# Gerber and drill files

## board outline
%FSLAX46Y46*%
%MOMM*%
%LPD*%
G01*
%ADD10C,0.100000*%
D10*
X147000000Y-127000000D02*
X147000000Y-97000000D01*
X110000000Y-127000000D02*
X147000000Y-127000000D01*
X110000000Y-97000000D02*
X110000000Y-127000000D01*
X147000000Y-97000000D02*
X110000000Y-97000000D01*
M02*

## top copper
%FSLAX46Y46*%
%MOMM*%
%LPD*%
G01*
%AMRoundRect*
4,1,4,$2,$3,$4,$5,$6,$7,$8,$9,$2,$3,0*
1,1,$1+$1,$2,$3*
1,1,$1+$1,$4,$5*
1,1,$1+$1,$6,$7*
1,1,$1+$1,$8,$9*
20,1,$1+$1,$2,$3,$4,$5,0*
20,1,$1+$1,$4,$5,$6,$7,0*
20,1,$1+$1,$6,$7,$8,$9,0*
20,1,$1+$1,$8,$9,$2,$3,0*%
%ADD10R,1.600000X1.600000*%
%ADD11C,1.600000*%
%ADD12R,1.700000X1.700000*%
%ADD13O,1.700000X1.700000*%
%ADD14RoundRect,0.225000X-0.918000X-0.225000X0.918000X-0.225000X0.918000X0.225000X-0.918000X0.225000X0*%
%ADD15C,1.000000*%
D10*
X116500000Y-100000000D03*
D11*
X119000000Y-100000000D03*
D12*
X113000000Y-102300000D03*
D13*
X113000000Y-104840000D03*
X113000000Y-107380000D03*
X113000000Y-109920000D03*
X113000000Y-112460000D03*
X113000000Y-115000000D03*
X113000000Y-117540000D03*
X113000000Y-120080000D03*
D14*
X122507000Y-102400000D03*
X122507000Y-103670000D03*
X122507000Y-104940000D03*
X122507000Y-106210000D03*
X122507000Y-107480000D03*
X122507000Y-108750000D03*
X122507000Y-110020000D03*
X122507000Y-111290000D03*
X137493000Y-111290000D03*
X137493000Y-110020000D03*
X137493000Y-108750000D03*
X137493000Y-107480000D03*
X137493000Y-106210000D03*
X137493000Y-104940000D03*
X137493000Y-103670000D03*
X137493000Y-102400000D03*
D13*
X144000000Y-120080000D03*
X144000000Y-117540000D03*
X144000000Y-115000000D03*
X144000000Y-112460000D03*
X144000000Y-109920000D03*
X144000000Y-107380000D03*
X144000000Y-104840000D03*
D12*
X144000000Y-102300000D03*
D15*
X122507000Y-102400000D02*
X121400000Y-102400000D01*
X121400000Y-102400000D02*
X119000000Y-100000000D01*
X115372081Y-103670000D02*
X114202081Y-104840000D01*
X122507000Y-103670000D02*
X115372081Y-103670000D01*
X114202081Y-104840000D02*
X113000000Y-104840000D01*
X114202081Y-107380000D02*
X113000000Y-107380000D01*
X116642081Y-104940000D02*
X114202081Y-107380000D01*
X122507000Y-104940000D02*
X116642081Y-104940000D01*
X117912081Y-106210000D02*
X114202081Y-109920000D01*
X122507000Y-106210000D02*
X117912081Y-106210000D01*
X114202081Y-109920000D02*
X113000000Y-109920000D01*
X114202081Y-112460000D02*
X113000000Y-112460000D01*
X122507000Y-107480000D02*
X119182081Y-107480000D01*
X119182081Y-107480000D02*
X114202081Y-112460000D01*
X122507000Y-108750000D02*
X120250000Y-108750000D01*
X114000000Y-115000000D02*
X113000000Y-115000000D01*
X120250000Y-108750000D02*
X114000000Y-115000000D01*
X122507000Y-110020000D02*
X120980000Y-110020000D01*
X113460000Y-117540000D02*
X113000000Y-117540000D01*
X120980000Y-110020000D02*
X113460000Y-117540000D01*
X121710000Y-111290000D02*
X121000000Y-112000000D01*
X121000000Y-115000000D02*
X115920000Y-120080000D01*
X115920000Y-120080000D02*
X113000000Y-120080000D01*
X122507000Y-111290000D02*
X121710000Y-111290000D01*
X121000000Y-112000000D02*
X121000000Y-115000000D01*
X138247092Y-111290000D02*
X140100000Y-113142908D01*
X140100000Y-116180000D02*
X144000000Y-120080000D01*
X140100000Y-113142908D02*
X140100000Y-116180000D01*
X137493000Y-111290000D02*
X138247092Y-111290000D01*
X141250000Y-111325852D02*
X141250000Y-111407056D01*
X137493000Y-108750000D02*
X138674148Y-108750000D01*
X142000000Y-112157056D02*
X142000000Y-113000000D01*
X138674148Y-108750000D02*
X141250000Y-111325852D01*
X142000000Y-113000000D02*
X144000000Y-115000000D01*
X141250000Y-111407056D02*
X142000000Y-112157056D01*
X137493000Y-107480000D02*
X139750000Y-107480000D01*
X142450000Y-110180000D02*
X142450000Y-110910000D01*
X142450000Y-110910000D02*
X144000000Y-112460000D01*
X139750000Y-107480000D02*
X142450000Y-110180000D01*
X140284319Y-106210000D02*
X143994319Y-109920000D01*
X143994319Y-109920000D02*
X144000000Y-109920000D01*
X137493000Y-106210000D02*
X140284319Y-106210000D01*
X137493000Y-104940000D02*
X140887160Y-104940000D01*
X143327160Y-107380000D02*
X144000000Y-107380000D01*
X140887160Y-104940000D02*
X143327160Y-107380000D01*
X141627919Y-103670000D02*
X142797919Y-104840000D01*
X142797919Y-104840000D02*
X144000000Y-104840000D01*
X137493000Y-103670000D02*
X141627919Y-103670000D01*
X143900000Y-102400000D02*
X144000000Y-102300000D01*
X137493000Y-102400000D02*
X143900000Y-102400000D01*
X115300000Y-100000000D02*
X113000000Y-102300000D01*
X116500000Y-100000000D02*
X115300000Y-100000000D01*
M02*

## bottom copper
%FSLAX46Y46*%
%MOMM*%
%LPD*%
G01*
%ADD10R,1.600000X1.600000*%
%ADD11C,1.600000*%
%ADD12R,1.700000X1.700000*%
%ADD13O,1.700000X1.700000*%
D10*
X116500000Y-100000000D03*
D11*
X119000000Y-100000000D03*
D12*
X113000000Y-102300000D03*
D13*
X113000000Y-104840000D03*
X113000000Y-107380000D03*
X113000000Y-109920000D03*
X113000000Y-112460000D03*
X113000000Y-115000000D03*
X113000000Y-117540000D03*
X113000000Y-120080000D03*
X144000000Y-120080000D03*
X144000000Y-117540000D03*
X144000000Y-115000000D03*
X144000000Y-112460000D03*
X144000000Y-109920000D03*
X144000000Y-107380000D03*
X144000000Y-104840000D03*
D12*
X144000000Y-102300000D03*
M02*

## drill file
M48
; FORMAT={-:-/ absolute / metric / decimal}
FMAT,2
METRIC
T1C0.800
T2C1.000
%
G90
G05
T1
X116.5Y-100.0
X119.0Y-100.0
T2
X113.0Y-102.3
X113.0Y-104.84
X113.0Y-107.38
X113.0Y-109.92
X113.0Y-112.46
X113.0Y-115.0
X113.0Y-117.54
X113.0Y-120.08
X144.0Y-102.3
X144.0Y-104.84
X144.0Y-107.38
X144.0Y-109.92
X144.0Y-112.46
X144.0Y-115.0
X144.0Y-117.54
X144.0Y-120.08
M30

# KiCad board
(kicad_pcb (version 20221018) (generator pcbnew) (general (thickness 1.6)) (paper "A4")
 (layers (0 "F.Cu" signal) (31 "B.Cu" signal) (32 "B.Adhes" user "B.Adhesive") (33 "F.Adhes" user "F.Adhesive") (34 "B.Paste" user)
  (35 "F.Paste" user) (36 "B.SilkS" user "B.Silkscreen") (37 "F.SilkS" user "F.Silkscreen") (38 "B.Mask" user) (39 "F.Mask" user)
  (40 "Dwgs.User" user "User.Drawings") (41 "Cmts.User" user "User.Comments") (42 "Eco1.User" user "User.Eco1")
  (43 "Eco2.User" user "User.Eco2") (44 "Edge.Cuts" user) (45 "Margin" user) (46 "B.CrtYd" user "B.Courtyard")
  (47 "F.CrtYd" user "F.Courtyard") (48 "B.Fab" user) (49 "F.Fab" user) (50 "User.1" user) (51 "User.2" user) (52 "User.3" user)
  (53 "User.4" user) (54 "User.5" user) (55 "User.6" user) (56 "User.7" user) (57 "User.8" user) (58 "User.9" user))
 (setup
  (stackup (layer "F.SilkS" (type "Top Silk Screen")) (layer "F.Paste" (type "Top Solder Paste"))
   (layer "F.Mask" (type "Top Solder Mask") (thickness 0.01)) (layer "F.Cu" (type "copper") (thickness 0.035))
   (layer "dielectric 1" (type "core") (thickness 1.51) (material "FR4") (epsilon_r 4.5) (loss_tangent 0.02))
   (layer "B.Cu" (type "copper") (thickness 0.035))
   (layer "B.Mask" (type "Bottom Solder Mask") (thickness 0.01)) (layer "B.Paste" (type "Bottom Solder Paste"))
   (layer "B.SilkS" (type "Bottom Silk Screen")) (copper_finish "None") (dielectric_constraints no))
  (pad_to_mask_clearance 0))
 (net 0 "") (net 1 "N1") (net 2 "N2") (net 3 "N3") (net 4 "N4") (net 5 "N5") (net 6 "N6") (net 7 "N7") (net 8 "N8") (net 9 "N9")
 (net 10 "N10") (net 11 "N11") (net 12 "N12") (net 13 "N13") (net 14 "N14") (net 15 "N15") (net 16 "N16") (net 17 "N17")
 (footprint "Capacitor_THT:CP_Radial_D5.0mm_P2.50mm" (layer "F.Cu") (at 116.5 100)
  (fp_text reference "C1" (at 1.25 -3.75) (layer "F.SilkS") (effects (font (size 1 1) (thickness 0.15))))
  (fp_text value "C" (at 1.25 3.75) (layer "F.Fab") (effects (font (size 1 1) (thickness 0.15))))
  (pad "1" thru_hole rect (at 0 0) (size 1.6 1.6) (drill 0.8) (layers "*.Cu" "*.Mask") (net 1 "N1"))
  (pad "2" thru_hole circle (at 2.5 0) (size 1.6 1.6) (drill 0.8) (layers "*.Cu" "*.Mask") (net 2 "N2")))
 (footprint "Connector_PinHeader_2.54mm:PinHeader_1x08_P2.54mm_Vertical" (layer "F.Cu") (at 113 102.3)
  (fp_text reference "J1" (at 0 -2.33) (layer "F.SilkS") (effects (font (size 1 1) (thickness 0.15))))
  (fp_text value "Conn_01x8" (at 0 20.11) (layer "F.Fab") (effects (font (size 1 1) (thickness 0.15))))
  (pad "1" thru_hole rect (at 0 0) (size 1.7 1.7) (drill 1) (layers "*.Cu" "*.Mask") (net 1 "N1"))
  (pad "2" thru_hole oval (at 0 2.54) (size 1.7 1.7) (drill 1) (layers "*.Cu" "*.Mask") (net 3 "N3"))
  (pad "3" thru_hole oval (at 0 5.08) (size 1.7 1.7) (drill 1) (layers "*.Cu" "*.Mask") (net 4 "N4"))
  (pad "4" thru_hole oval (at 0 7.62) (size 1.7 1.7) (drill 1) (layers "*.Cu" "*.Mask") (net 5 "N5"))
  (pad "5" thru_hole oval (at 0 10.16) (size 1.7 1.7) (drill 1) (layers "*.Cu" "*.Mask") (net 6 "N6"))
  (pad "6" thru_hole oval (at 0 12.7) (size 1.7 1.7) (drill 1) (layers "*.Cu" "*.Mask") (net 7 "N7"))
  (pad "7" thru_hole oval (at 0 15.24) (size 1.7 1.7) (drill 1) (layers "*.Cu" "*.Mask") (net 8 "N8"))
  (pad "8" thru_hole oval (at 0 17.78) (size 1.7 1.7) (drill 1) (layers "*.Cu" "*.Mask") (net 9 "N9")))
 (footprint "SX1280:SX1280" (layer "F.Cu") (at 130.493 95.52)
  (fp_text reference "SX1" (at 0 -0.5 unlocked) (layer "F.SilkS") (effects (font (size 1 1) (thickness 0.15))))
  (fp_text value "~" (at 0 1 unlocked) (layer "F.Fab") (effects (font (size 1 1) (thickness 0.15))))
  (pad "1" smd roundrect (at -7.986 6.88) (size 2.286 0.9) (layers "F.Cu" "F.Paste" "F.Mask") (roundrect_rratio 0.25) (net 2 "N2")
   (thermal_bridge_angle 45))
  (pad "2" smd roundrect (at -7.986 8.15) (size 2.286 0.9) (layers "F.Cu" "F.Paste" "F.Mask") (roundrect_rratio 0.25) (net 3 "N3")
   (thermal_bridge_angle 45))
  (pad "3" smd roundrect (at -7.986 9.42) (size 2.286 0.9) (layers "F.Cu" "F.Paste" "F.Mask") (roundrect_rratio 0.25) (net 4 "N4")
   (thermal_bridge_angle 45))
  (pad "4" smd roundrect (at -7.986 10.69) (size 2.286 0.9) (layers "F.Cu" "F.Paste" "F.Mask") (roundrect_rratio 0.25) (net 5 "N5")
   (thermal_bridge_angle 45))
  (pad "5" smd roundrect (at -7.986 11.96) (size 2.286 0.9) (layers "F.Cu" "F.Paste" "F.Mask") (roundrect_rratio 0.25) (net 6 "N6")
   (thermal_bridge_angle 45))
  (pad "6" smd roundrect (at -7.986 13.23) (size 2.286 0.9) (layers "F.Cu" "F.Paste" "F.Mask") (roundrect_rratio 0.25) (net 7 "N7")
   (thermal_bridge_angle 45))
  (pad "7" smd roundrect (at -7.986 14.5) (size 2.286 0.9) (layers "F.Cu" "F.Paste" "F.Mask") (roundrect_rratio 0.25) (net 8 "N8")
   (thermal_bridge_angle 45))
  (pad "8" smd roundrect (at -7.986 15.77) (size 2.286 0.9) (layers "F.Cu" "F.Paste" "F.Mask") (roundrect_rratio 0.25) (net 9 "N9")
   (thermal_bridge_angle 45))
  (pad "9" smd roundrect (at 7 15.77) (size 2.286 0.9) (layers "F.Cu" "F.Paste" "F.Mask") (roundrect_rratio 0.25) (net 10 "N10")
   (thermal_bridge_angle 45))
  (pad "10" smd roundrect (at 7 14.5) (size 2.286 0.9) (layers "F.Cu" "F.Paste" "F.Mask") (roundrect_rratio 0.25) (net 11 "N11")
   (thermal_bridge_angle 45))
  (pad "11" smd roundrect (at 7 13.23) (size 2.286 0.9) (layers "F.Cu" "F.Paste" "F.Mask") (roundrect_rratio 0.25) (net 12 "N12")
   (thermal_bridge_angle 45))
  (pad "12" smd roundrect (at 7 11.96) (size 2.286 0.9) (layers "F.Cu" "F.Paste" "F.Mask") (roundrect_rratio 0.25) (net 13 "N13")
   (thermal_bridge_angle 45))
  (pad "13" smd roundrect (at 7 10.69) (size 2.286 0.9) (layers "F.Cu" "F.Paste" "F.Mask") (roundrect_rratio 0.25) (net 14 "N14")
   (thermal_bridge_angle 45))
  (pad "14" smd roundrect (at 7 9.42) (size 2.286 0.9) (layers "F.Cu" "F.Paste" "F.Mask") (roundrect_rratio 0.25) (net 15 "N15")
   (thermal_bridge_angle 45))
  (pad "15" smd roundrect (at 7 8.15) (size 2.286 0.9) (layers "F.Cu" "F.Paste" "F.Mask") (roundrect_rratio 0.25) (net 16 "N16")
   (thermal_bridge_angle 45))
  (pad "16" smd roundrect (at 7 6.88) (size 2.286 0.9) (layers "F.Cu" "F.Paste" "F.Mask") (roundrect_rratio 0.25) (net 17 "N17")
   (thermal_bridge_angle 45)))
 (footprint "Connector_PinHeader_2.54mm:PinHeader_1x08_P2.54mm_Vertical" (layer "F.Cu") (at 144 102.3)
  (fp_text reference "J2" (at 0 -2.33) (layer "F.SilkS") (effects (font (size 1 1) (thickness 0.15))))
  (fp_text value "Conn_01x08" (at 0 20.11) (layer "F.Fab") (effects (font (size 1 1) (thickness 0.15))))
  (pad "9" thru_hole oval (at 0 17.78) (size 1.7 1.7) (drill 1) (layers "*.Cu" "*.Mask") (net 10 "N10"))
  (pad "10" thru_hole oval (at 0 15.24) (size 1.7 1.7) (drill 1) (layers "*.Cu" "*.Mask") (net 11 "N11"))
  (pad "11" thru_hole oval (at 0 12.7) (size 1.7 1.7) (drill 1) (layers "*.Cu" "*.Mask") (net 12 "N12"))
  (pad "12" thru_hole oval (at 0 10.16) (size 1.7 1.7) (drill 1) (layers "*.Cu" "*.Mask") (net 13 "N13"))
  (pad "13" thru_hole oval (at 0 7.62) (size 1.7 1.7) (drill 1) (layers "*.Cu" "*.Mask") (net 14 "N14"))
  (pad "14" thru_hole oval (at 0 5.08) (size 1.7 1.7) (drill 1) (layers "*.Cu" "*.Mask") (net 15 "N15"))
  (pad "15" thru_hole oval (at 0 2.54) (size 1.7 1.7) (drill 1) (layers "*.Cu" "*.Mask") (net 16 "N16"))
  (pad "16" thru_hole rect (at 0 0) (size 1.7 1.7) (drill 1) (layers "*.Cu" "*.Mask") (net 17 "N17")))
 (gr_line (start 147 127) (end 147 97) (stroke (width 0.1) (type default)) (layer "Edge.Cuts"))
 (gr_line (start 110 127) (end 147 127) (stroke (width 0.1) (type default)) (layer "Edge.Cuts"))
 (gr_line (start 110 97) (end 110 127) (stroke (width 0.1) (type default)) (layer "Edge.Cuts"))
 (gr_line (start 147 97) (end 110 97) (stroke (width 0.1) (type default)) (layer "Edge.Cuts"))
 (segment (start 122.507 102.4) (end 121.4 102.4) (width 1) (layer "F.Cu") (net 2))
 (segment (start 121.4 102.4) (end 119 100) (width 1) (layer "F.Cu") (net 2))
 (segment (start 115.372081 103.67) (end 114.202081 104.84) (width 1) (layer "F.Cu") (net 3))
 (segment (start 122.507 103.67) (end 115.372081 103.67) (width 1) (layer "F.Cu") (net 3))
 (segment (start 114.202081 104.84) (end 113 104.84) (width 1) (layer "F.Cu") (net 3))
 (segment (start 114.202081 107.38) (end 113 107.38) (width 1) (layer "F.Cu") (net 4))
 (segment (start 116.642081 104.94) (end 114.202081 107.38) (width 1) (layer "F.Cu") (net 4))
 (segment (start 122.507 104.94) (end 116.642081 104.94) (width 1) (layer "F.Cu") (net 4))
 (segment (start 117.912081 106.21) (end 114.202081 109.92) (width 1) (layer "F.Cu") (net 5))
 (segment (start 122.507 106.21) (end 117.912081 106.21) (width 1) (layer "F.Cu") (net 5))
 (segment (start 114.202081 109.92) (end 113 109.92) (width 1) (layer "F.Cu") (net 5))
 (segment (start 114.202081 112.46) (end 113 112.46) (width 1) (layer "F.Cu") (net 6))
 (segment (start 122.507 107.48) (end 119.182081 107.48) (width 1) (layer "F.Cu") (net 6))
 (segment (start 119.182081 107.48) (end 114.202081 112.46) (width 1) (layer "F.Cu") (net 6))
 (segment (start 122.507 108.75) (end 120.25 108.75) (width 1) (layer "F.Cu") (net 7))
 (segment (start 114 115) (end 113 115) (width 1) (layer "F.Cu") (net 7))
 (segment (start 120.25 108.75) (end 114 115) (width 1) (layer "F.Cu") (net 7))
 (segment (start 122.507 110.02) (end 120.98 110.02) (width 1) (layer "F.Cu") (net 8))
 (segment (start 113.46 117.54) (end 113 117.54) (width 1) (layer "F.Cu") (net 8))
 (segment (start 120.98 110.02) (end 113.46 117.54) (width 1) (layer "F.Cu") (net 8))
 (segment (start 121.71 111.29) (end 121 112) (width 1) (layer "F.Cu") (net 9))
 (segment (start 121 115) (end 115.92 120.08) (width 1) (layer "F.Cu") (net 9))
 (segment (start 115.92 120.08) (end 113 120.08) (width 1) (layer "F.Cu") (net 9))
 (segment (start 122.507 111.29) (end 121.71 111.29) (width 1) (layer "F.Cu") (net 9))
 (segment (start 121 112) (end 121 115) (width 1) (layer "F.Cu") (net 9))
 (segment (start 138.247092 111.29) (end 140.1 113.142908) (width 1) (layer "F.Cu") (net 10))
 (segment (start 140.1 116.18) (end 144 120.08) (width 1) (layer "F.Cu") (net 10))
 (segment (start 140.1 113.142908) (end 140.1 116.18) (width 1) (layer "F.Cu") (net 10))
 (segment (start 137.493 111.29) (end 138.247092 111.29) (width 1) (layer "F.Cu") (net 10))
 (segment (start 141.25 111.325852) (end 141.25 111.407056) (width 1) (layer "F.Cu") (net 12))
 (segment (start 137.493 108.75) (end 138.674148 108.75) (width 1) (layer "F.Cu") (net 12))
 (segment (start 142 112.157056) (end 142 113) (width 1) (layer "F.Cu") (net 12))
 (segment (start 138.674148 108.75) (end 141.25 111.325852) (width 1) (layer "F.Cu") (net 12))
 (segment (start 142 113) (end 144 115) (width 1) (layer "F.Cu") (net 12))
 (segment (start 141.25 111.407056) (end 142 112.157056) (width 1) (layer "F.Cu") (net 12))
 (segment (start 137.493 107.48) (end 139.75 107.48) (width 1) (layer "F.Cu") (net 13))
 (segment (start 142.45 110.18) (end 142.45 110.91) (width 1) (layer "F.Cu") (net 13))
 (segment (start 142.45 110.91) (end 144 112.46) (width 1) (layer "F.Cu") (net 13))
 (segment (start 139.75 107.48) (end 142.45 110.18) (width 1) (layer "F.Cu") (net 13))
 (segment (start 140.284319 106.21) (end 143.994319 109.92) (width 1) (layer "F.Cu") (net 14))
 (segment (start 143.994319 109.92) (end 144 109.92) (width 1) (layer "F.Cu") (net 14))
 (segment (start 137.493 106.21) (end 140.284319 106.21) (width 1) (layer "F.Cu") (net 14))
 (segment (start 137.493 104.94) (end 140.88716 104.94) (width 1) (layer "F.Cu") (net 15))
 (segment (start 143.32716 107.38) (end 144 107.38) (width 1) (layer "F.Cu") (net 15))
 (segment (start 140.88716 104.94) (end 143.32716 107.38) (width 1) (layer "F.Cu") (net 15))
 (segment (start 141.627919 103.67) (end 142.797919 104.84) (width 1) (layer "F.Cu") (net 16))
 (segment (start 142.797919 104.84) (end 144 104.84) (width 1) (layer "F.Cu") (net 16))
 (segment (start 137.493 103.67) (end 141.627919 103.67) (width 1) (layer "F.Cu") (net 16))
 (segment (start 143.9 102.4) (end 144 102.3) (width 1) (layer "F.Cu") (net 17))
 (segment (start 137.493 102.4) (end 143.9 102.4) (width 1) (layer "F.Cu") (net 17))
 (segment (start 115.3 100) (end 113 102.3) (width 1) (layer "F.Cu") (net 1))
 (segment (start 116.5 100) (end 115.3 100) (width 1) (layer "F.Cu") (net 1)))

